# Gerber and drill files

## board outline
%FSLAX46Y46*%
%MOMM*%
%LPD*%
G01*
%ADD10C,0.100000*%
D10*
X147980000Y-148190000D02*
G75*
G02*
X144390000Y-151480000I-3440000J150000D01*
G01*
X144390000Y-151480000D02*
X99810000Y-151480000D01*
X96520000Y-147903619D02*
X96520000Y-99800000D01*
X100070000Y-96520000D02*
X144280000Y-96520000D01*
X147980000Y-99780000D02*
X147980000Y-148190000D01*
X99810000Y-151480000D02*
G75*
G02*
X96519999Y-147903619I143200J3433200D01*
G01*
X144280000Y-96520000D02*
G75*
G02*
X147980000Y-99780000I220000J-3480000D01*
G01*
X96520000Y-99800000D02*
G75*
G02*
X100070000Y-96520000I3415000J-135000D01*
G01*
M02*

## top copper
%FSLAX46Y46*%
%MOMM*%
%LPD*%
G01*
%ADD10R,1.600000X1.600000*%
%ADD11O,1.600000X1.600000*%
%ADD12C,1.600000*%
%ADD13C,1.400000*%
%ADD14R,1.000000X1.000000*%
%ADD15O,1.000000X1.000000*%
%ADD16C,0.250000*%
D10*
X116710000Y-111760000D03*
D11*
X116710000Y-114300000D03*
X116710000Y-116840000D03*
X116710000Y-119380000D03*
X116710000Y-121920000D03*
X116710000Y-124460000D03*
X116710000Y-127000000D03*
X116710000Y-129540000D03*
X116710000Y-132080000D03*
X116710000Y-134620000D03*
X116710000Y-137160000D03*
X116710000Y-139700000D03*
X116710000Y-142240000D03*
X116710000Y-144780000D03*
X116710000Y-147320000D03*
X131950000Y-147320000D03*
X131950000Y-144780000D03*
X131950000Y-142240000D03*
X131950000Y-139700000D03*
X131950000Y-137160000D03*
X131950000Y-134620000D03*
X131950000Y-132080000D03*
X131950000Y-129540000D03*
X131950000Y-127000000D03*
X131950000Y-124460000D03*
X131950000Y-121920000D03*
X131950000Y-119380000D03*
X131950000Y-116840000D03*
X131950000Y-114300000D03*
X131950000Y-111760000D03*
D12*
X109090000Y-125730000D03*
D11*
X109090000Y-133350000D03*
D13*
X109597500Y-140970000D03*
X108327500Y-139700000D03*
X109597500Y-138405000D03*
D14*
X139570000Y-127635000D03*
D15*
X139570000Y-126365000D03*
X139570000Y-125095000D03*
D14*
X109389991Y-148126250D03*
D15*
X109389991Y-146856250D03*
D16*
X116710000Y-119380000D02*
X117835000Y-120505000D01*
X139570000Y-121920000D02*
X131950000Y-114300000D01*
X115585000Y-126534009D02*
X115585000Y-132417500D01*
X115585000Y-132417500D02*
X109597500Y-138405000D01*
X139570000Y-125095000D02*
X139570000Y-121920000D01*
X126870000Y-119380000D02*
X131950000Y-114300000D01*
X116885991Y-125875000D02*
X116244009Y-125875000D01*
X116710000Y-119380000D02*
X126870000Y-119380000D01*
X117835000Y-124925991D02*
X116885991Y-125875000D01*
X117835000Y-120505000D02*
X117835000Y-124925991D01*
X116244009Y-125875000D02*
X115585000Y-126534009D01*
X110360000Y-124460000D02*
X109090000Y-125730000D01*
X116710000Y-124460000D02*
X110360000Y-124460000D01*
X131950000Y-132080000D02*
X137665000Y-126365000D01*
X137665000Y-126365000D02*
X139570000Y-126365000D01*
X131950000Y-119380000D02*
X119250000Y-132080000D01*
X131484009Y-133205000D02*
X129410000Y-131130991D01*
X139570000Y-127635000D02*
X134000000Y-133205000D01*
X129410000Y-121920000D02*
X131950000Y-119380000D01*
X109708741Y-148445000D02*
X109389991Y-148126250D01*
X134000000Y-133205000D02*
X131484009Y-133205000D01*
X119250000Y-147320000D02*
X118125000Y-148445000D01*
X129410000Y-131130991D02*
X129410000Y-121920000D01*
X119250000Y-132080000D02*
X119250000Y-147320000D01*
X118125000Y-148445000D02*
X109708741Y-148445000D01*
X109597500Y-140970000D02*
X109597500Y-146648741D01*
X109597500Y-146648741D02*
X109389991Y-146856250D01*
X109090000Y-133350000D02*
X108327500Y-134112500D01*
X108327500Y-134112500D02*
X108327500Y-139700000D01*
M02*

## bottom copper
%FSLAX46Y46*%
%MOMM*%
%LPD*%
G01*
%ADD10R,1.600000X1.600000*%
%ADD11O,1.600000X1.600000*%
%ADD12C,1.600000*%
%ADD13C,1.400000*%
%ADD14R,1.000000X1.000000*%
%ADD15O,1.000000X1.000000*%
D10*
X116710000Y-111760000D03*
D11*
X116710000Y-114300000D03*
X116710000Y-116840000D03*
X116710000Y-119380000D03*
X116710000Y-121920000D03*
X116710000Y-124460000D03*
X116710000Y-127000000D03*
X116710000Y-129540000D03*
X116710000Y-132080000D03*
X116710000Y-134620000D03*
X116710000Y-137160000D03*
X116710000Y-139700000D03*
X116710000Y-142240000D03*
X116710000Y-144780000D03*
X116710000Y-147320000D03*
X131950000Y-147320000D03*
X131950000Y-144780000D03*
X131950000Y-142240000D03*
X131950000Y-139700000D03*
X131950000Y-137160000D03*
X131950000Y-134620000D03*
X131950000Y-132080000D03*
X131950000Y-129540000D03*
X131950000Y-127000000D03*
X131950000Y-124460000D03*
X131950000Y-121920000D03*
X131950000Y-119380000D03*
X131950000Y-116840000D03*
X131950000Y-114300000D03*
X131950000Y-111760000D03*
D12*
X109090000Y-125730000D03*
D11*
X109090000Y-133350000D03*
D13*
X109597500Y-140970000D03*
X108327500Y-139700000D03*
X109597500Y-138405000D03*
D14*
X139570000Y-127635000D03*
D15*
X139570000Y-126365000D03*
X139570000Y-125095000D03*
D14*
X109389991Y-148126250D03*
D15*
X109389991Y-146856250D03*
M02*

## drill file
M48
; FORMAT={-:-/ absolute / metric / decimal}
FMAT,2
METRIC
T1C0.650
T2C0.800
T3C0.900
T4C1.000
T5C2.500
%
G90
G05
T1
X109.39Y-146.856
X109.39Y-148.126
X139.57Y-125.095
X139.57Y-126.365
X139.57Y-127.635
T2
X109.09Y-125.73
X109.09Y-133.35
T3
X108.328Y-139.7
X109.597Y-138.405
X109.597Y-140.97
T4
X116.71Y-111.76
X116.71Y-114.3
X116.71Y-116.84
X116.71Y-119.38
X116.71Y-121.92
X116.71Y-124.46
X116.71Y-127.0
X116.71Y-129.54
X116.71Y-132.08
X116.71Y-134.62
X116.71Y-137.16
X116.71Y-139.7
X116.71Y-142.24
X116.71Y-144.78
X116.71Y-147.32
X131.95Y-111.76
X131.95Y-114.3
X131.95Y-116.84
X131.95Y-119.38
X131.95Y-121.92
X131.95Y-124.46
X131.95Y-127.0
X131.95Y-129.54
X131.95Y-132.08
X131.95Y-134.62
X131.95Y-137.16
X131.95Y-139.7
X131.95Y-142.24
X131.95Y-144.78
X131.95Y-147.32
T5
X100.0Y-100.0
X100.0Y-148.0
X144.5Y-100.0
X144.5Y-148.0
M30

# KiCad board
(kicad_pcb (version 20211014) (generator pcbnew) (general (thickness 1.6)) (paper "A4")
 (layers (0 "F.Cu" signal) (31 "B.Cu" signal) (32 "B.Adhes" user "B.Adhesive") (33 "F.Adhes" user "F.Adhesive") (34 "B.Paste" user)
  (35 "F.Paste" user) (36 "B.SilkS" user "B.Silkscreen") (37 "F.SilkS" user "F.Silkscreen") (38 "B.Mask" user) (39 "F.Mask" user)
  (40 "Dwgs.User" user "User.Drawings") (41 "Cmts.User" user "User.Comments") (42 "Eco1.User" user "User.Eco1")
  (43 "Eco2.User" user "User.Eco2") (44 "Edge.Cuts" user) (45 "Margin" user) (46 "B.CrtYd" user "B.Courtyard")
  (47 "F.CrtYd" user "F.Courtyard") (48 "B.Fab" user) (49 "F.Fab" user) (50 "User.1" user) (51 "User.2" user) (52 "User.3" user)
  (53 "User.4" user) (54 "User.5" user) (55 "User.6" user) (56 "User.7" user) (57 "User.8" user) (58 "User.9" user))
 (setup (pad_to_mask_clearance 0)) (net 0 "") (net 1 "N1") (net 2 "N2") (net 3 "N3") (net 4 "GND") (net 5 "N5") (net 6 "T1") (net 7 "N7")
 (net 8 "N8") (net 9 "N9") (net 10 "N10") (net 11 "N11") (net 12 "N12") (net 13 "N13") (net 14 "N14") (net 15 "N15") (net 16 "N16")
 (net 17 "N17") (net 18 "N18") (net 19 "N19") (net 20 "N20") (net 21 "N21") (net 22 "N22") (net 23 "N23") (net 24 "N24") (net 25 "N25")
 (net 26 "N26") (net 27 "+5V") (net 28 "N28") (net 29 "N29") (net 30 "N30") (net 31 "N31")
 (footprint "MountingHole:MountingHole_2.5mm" (layer "F.Cu") (at 144.5 148)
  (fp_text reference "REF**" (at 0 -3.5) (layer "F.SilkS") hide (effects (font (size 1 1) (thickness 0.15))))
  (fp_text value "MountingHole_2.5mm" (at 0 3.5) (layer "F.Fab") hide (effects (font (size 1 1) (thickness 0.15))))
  (pad "" np_thru_hole circle (at 0 0) (size 2.5 2.5) (drill 2.5) (layers F&B.Cu *.Mask)))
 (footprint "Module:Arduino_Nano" (layer "F.Cu") (at 116.71 111.76)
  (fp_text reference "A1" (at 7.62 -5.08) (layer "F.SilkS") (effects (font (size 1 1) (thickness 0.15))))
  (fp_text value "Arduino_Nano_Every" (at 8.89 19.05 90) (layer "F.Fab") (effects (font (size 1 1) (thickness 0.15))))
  (pad "1" thru_hole rect (at 0 0) (size 1.6 1.6) (drill 1) (layers *.Cu *.Mask) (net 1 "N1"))
  (pad "2" thru_hole oval (at 0 2.54) (size 1.6 1.6) (drill 1) (layers *.Cu *.Mask) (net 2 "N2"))
  (pad "3" thru_hole oval (at 0 5.08) (size 1.6 1.6) (drill 1) (layers *.Cu *.Mask) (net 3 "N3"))
  (pad "4" thru_hole oval (at 0 7.62) (size 1.6 1.6) (drill 1) (layers *.Cu *.Mask) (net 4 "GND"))
  (pad "5" thru_hole oval (at 0 10.16) (size 1.6 1.6) (drill 1) (layers *.Cu *.Mask) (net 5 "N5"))
  (pad "6" thru_hole oval (at 0 12.7) (size 1.6 1.6) (drill 1) (layers *.Cu *.Mask) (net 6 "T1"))
  (pad "7" thru_hole oval (at 0 15.24) (size 1.6 1.6) (drill 1) (layers *.Cu *.Mask) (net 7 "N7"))
  (pad "8" thru_hole oval (at 0 17.78) (size 1.6 1.6) (drill 1) (layers *.Cu *.Mask) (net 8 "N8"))
  (pad "9" thru_hole oval (at 0 20.32) (size 1.6 1.6) (drill 1) (layers *.Cu *.Mask) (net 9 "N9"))
  (pad "10" thru_hole oval (at 0 22.86) (size 1.6 1.6) (drill 1) (layers *.Cu *.Mask) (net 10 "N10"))
  (pad "11" thru_hole oval (at 0 25.4) (size 1.6 1.6) (drill 1) (layers *.Cu *.Mask) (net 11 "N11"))
  (pad "12" thru_hole oval (at 0 27.94) (size 1.6 1.6) (drill 1) (layers *.Cu *.Mask) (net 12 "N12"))
  (pad "13" thru_hole oval (at 0 30.48) (size 1.6 1.6) (drill 1) (layers *.Cu *.Mask) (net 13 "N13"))
  (pad "14" thru_hole oval (at 0 33.02) (size 1.6 1.6) (drill 1) (layers *.Cu *.Mask) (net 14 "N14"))
  (pad "15" thru_hole oval (at 0 35.56) (size 1.6 1.6) (drill 1) (layers *.Cu *.Mask) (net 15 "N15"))
  (pad "16" thru_hole oval (at 15.24 35.56) (size 1.6 1.6) (drill 1) (layers *.Cu *.Mask) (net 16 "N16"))
  (pad "17" thru_hole oval (at 15.24 33.02) (size 1.6 1.6) (drill 1) (layers *.Cu *.Mask) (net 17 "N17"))
  (pad "18" thru_hole oval (at 15.24 30.48) (size 1.6 1.6) (drill 1) (layers *.Cu *.Mask) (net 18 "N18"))
  (pad "19" thru_hole oval (at 15.24 27.94) (size 1.6 1.6) (drill 1) (layers *.Cu *.Mask) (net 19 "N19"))
  (pad "20" thru_hole oval (at 15.24 25.4) (size 1.6 1.6) (drill 1) (layers *.Cu *.Mask) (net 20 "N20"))
  (pad "21" thru_hole oval (at 15.24 22.86) (size 1.6 1.6) (drill 1) (layers *.Cu *.Mask) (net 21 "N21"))
  (pad "22" thru_hole oval (at 15.24 20.32) (size 1.6 1.6) (drill 1) (layers *.Cu *.Mask) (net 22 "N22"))
  (pad "23" thru_hole oval (at 15.24 17.78) (size 1.6 1.6) (drill 1) (layers *.Cu *.Mask) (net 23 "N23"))
  (pad "24" thru_hole oval (at 15.24 15.24) (size 1.6 1.6) (drill 1) (layers *.Cu *.Mask) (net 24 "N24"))
  (pad "25" thru_hole oval (at 15.24 12.7) (size 1.6 1.6) (drill 1) (layers *.Cu *.Mask) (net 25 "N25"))
  (pad "26" thru_hole oval (at 15.24 10.16) (size 1.6 1.6) (drill 1) (layers *.Cu *.Mask) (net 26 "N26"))
  (pad "27" thru_hole oval (at 15.24 7.62) (size 1.6 1.6) (drill 1) (layers *.Cu *.Mask) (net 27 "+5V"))
  (pad "28" thru_hole oval (at 15.24 5.08) (size 1.6 1.6) (drill 1) (layers *.Cu *.Mask) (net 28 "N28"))
  (pad "29" thru_hole oval (at 15.24 2.54) (size 1.6 1.6) (drill 1) (layers *.Cu *.Mask) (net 4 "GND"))
  (pad "30" thru_hole oval (at 15.24 0) (size 1.6 1.6) (drill 1) (layers *.Cu *.Mask) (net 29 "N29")))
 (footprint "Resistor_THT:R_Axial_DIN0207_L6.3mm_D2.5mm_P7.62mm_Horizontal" (layer "F.Cu") (at 109.09 125.73 -90)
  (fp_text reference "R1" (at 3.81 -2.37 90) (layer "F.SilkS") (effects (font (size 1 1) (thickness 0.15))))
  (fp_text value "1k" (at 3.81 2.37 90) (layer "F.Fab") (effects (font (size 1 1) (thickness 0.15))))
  (pad "1" thru_hole circle (at 0 0 270) (size 1.6 1.6) (drill 0.8) (layers *.Cu *.Mask) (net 6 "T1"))
  (pad "2" thru_hole oval (at 7.62 0 270) (size 1.6 1.6) (drill 0.8) (layers *.Cu *.Mask) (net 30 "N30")))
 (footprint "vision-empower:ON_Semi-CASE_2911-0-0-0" (layer "F.Cu") (at 109.09 139.7)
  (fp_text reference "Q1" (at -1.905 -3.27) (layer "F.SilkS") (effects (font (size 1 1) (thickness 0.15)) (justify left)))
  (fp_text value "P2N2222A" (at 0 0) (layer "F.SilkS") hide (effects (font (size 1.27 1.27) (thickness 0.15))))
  (pad "1" thru_hole circle (at 0.5075 1.27) (size 1.4 1.4) (drill 0.9) (layers *.Cu) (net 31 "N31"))
  (pad "2" thru_hole circle (at -0.7625 0) (size 1.4 1.4) (drill 0.9) (layers *.Cu) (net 30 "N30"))
  (pad "3" thru_hole circle (at 0.5075 -1.295) (size 1.4 1.4) (drill 0.9) (layers *.Cu) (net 4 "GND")))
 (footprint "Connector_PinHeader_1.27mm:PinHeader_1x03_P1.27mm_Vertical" (layer "F.Cu") (at 139.57 127.635 180)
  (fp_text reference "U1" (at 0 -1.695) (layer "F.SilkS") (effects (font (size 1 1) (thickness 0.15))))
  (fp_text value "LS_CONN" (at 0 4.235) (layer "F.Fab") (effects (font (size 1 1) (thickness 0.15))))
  (pad "1" thru_hole rect (at 0 0 180) (size 1 1) (drill 0.65) (layers *.Cu *.Mask) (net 27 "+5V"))
  (pad "2" thru_hole oval (at 0 1.27 180) (size 1 1) (drill 0.65) (layers *.Cu *.Mask) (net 22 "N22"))
  (pad "3" thru_hole oval (at 0 2.54 180) (size 1 1) (drill 0.65) (layers *.Cu *.Mask) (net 4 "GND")))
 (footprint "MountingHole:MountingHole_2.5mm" (layer "F.Cu") (at 100 148)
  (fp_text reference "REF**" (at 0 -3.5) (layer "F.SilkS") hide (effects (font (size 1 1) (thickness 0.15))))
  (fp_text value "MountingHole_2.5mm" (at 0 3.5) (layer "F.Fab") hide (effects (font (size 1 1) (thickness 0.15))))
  (pad "" np_thru_hole circle (at 0 0) (size 2.5 2.5) (drill 2.5) (layers F&B.Cu *.Mask)))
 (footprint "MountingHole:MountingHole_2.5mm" (layer "F.Cu") (at 144.5 100)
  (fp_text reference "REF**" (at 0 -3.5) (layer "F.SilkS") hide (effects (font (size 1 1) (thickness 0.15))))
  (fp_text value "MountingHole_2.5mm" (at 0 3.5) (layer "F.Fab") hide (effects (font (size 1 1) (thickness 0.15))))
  (pad "" np_thru_hole circle (at 0 0) (size 2.5 2.5) (drill 2.5) (layers F&B.Cu *.Mask)))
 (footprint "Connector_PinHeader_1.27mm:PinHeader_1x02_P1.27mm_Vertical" (layer "F.Cu") (at 109.389991 148.12625 180)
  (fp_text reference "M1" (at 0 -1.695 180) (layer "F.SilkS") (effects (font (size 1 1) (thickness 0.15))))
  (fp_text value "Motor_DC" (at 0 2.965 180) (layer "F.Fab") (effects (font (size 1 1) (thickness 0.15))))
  (pad "1" thru_hole rect (at 0 0 180) (size 1 1) (drill 0.65) (layers *.Cu *.Mask) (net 27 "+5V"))
  (pad "2" thru_hole oval (at 0 1.27 180) (size 1 1) (drill 0.65) (layers *.Cu *.Mask) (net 31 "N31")))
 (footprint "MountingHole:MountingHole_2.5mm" (layer "F.Cu") (at 100 100)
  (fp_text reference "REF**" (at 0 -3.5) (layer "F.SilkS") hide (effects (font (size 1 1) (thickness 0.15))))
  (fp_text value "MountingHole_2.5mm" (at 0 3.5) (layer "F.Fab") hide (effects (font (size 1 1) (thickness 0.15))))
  (pad "" np_thru_hole circle (at 0 0) (size 2.5 2.5) (drill 2.5) (layers *.Cu *.Mask)))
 (gr_arc (start 147.98 148.19) (mid 146.866381 150.578513) (end 144.39 151.48) (layer "Edge.Cuts") (width 0.1))
 (gr_line (start 144.39 151.48) (end 99.81 151.48) (layer "Edge.Cuts") (width 0.1))
 (gr_line (start 96.52 147.903619) (end 96.52 99.8) (layer "Edge.Cuts") (width 0.1))
 (gr_line (start 100.07 96.52) (end 144.28 96.52) (layer "Edge.Cuts") (width 0.1))
 (gr_line (start 147.98 99.78) (end 147.98 148.19) (layer "Edge.Cuts") (width 0.1))
 (gr_arc (start 99.81 151.48) (mid 97.424308 150.373191) (end 96.52 147.903619) (layer "Edge.Cuts") (width 0.1))
 (gr_arc (start 144.28 96.52) (mid 146.805168 97.383705) (end 147.98 99.78) (layer "Edge.Cuts") (width 0.1))
 (gr_arc (start 96.52 99.8) (mid 97.61569 97.424771) (end 100.07 96.52) (layer "Edge.Cuts") (width 0.1))
 (segment (start 116.71 119.38) (end 117.835 120.505) (width 0.25) (layer "F.Cu") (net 4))
 (segment (start 139.57 121.92) (end 131.95 114.3) (width 0.25) (layer "F.Cu") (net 4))
 (segment (start 115.585 126.534009) (end 115.585 132.4175) (width 0.25) (layer "F.Cu") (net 4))
 (segment (start 115.585 132.4175) (end 109.5975 138.405) (width 0.25) (layer "F.Cu") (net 4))
 (segment (start 139.57 125.095) (end 139.57 121.92) (width 0.25) (layer "F.Cu") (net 4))
 (segment (start 126.87 119.38) (end 131.95 114.3) (width 0.25) (layer "F.Cu") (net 4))
 (segment (start 116.885991 125.875) (end 116.244009 125.875) (width 0.25) (layer "F.Cu") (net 4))
 (segment (start 116.71 119.38) (end 126.87 119.38) (width 0.25) (layer "F.Cu") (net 4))
 (segment (start 117.835 124.925991) (end 116.885991 125.875) (width 0.25) (layer "F.Cu") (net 4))
 (segment (start 117.835 120.505) (end 117.835 124.925991) (width 0.25) (layer "F.Cu") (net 4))
 (segment (start 116.244009 125.875) (end 115.585 126.534009) (width 0.25) (layer "F.Cu") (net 4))
 (segment (start 110.36 124.46) (end 109.09 125.73) (width 0.25) (layer "F.Cu") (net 6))
 (segment (start 116.71 124.46) (end 110.36 124.46) (width 0.25) (layer "F.Cu") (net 6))
 (segment (start 131.95 132.08) (end 137.665 126.365) (width 0.25) (layer "F.Cu") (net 22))
 (segment (start 137.665 126.365) (end 139.57 126.365) (width 0.25) (layer "F.Cu") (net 22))
 (segment (start 131.95 119.38) (end 119.25 132.08) (width 0.25) (layer "F.Cu") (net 27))
 (segment (start 131.484009 133.205) (end 129.41 131.130991) (width 0.25) (layer "F.Cu") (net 27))
 (segment (start 139.57 127.635) (end 134 133.205) (width 0.25) (layer "F.Cu") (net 27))
 (segment (start 129.41 121.92) (end 131.95 119.38) (width 0.25) (layer "F.Cu") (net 27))
 (segment (start 109.708741 148.445) (end 109.389991 148.12625) (width 0.25) (layer "F.Cu") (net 27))
 (segment (start 134 133.205) (end 131.484009 133.205) (width 0.25) (layer "F.Cu") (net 27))
 (segment (start 119.25 147.32) (end 118.125 148.445) (width 0.25) (layer "F.Cu") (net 27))
 (segment (start 129.41 131.130991) (end 129.41 121.92) (width 0.25) (layer "F.Cu") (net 27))
 (segment (start 119.25 132.08) (end 119.25 147.32) (width 0.25) (layer "F.Cu") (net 27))
 (segment (start 118.125 148.445) (end 109.708741 148.445) (width 0.25) (layer "F.Cu") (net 27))
 (segment (start 109.5975 140.97) (end 109.5975 146.648741) (width 0.25) (layer "F.Cu") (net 31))
 (segment (start 109.5975 146.648741) (end 109.389991 146.85625) (width 0.25) (layer "F.Cu") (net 31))
 (segment (start 109.09 133.35) (end 108.3275 134.1125) (width 0.25) (layer "F.Cu") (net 30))
 (segment (start 108.3275 134.1125) (end 108.3275 139.7) (width 0.25) (layer "F.Cu") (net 30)))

